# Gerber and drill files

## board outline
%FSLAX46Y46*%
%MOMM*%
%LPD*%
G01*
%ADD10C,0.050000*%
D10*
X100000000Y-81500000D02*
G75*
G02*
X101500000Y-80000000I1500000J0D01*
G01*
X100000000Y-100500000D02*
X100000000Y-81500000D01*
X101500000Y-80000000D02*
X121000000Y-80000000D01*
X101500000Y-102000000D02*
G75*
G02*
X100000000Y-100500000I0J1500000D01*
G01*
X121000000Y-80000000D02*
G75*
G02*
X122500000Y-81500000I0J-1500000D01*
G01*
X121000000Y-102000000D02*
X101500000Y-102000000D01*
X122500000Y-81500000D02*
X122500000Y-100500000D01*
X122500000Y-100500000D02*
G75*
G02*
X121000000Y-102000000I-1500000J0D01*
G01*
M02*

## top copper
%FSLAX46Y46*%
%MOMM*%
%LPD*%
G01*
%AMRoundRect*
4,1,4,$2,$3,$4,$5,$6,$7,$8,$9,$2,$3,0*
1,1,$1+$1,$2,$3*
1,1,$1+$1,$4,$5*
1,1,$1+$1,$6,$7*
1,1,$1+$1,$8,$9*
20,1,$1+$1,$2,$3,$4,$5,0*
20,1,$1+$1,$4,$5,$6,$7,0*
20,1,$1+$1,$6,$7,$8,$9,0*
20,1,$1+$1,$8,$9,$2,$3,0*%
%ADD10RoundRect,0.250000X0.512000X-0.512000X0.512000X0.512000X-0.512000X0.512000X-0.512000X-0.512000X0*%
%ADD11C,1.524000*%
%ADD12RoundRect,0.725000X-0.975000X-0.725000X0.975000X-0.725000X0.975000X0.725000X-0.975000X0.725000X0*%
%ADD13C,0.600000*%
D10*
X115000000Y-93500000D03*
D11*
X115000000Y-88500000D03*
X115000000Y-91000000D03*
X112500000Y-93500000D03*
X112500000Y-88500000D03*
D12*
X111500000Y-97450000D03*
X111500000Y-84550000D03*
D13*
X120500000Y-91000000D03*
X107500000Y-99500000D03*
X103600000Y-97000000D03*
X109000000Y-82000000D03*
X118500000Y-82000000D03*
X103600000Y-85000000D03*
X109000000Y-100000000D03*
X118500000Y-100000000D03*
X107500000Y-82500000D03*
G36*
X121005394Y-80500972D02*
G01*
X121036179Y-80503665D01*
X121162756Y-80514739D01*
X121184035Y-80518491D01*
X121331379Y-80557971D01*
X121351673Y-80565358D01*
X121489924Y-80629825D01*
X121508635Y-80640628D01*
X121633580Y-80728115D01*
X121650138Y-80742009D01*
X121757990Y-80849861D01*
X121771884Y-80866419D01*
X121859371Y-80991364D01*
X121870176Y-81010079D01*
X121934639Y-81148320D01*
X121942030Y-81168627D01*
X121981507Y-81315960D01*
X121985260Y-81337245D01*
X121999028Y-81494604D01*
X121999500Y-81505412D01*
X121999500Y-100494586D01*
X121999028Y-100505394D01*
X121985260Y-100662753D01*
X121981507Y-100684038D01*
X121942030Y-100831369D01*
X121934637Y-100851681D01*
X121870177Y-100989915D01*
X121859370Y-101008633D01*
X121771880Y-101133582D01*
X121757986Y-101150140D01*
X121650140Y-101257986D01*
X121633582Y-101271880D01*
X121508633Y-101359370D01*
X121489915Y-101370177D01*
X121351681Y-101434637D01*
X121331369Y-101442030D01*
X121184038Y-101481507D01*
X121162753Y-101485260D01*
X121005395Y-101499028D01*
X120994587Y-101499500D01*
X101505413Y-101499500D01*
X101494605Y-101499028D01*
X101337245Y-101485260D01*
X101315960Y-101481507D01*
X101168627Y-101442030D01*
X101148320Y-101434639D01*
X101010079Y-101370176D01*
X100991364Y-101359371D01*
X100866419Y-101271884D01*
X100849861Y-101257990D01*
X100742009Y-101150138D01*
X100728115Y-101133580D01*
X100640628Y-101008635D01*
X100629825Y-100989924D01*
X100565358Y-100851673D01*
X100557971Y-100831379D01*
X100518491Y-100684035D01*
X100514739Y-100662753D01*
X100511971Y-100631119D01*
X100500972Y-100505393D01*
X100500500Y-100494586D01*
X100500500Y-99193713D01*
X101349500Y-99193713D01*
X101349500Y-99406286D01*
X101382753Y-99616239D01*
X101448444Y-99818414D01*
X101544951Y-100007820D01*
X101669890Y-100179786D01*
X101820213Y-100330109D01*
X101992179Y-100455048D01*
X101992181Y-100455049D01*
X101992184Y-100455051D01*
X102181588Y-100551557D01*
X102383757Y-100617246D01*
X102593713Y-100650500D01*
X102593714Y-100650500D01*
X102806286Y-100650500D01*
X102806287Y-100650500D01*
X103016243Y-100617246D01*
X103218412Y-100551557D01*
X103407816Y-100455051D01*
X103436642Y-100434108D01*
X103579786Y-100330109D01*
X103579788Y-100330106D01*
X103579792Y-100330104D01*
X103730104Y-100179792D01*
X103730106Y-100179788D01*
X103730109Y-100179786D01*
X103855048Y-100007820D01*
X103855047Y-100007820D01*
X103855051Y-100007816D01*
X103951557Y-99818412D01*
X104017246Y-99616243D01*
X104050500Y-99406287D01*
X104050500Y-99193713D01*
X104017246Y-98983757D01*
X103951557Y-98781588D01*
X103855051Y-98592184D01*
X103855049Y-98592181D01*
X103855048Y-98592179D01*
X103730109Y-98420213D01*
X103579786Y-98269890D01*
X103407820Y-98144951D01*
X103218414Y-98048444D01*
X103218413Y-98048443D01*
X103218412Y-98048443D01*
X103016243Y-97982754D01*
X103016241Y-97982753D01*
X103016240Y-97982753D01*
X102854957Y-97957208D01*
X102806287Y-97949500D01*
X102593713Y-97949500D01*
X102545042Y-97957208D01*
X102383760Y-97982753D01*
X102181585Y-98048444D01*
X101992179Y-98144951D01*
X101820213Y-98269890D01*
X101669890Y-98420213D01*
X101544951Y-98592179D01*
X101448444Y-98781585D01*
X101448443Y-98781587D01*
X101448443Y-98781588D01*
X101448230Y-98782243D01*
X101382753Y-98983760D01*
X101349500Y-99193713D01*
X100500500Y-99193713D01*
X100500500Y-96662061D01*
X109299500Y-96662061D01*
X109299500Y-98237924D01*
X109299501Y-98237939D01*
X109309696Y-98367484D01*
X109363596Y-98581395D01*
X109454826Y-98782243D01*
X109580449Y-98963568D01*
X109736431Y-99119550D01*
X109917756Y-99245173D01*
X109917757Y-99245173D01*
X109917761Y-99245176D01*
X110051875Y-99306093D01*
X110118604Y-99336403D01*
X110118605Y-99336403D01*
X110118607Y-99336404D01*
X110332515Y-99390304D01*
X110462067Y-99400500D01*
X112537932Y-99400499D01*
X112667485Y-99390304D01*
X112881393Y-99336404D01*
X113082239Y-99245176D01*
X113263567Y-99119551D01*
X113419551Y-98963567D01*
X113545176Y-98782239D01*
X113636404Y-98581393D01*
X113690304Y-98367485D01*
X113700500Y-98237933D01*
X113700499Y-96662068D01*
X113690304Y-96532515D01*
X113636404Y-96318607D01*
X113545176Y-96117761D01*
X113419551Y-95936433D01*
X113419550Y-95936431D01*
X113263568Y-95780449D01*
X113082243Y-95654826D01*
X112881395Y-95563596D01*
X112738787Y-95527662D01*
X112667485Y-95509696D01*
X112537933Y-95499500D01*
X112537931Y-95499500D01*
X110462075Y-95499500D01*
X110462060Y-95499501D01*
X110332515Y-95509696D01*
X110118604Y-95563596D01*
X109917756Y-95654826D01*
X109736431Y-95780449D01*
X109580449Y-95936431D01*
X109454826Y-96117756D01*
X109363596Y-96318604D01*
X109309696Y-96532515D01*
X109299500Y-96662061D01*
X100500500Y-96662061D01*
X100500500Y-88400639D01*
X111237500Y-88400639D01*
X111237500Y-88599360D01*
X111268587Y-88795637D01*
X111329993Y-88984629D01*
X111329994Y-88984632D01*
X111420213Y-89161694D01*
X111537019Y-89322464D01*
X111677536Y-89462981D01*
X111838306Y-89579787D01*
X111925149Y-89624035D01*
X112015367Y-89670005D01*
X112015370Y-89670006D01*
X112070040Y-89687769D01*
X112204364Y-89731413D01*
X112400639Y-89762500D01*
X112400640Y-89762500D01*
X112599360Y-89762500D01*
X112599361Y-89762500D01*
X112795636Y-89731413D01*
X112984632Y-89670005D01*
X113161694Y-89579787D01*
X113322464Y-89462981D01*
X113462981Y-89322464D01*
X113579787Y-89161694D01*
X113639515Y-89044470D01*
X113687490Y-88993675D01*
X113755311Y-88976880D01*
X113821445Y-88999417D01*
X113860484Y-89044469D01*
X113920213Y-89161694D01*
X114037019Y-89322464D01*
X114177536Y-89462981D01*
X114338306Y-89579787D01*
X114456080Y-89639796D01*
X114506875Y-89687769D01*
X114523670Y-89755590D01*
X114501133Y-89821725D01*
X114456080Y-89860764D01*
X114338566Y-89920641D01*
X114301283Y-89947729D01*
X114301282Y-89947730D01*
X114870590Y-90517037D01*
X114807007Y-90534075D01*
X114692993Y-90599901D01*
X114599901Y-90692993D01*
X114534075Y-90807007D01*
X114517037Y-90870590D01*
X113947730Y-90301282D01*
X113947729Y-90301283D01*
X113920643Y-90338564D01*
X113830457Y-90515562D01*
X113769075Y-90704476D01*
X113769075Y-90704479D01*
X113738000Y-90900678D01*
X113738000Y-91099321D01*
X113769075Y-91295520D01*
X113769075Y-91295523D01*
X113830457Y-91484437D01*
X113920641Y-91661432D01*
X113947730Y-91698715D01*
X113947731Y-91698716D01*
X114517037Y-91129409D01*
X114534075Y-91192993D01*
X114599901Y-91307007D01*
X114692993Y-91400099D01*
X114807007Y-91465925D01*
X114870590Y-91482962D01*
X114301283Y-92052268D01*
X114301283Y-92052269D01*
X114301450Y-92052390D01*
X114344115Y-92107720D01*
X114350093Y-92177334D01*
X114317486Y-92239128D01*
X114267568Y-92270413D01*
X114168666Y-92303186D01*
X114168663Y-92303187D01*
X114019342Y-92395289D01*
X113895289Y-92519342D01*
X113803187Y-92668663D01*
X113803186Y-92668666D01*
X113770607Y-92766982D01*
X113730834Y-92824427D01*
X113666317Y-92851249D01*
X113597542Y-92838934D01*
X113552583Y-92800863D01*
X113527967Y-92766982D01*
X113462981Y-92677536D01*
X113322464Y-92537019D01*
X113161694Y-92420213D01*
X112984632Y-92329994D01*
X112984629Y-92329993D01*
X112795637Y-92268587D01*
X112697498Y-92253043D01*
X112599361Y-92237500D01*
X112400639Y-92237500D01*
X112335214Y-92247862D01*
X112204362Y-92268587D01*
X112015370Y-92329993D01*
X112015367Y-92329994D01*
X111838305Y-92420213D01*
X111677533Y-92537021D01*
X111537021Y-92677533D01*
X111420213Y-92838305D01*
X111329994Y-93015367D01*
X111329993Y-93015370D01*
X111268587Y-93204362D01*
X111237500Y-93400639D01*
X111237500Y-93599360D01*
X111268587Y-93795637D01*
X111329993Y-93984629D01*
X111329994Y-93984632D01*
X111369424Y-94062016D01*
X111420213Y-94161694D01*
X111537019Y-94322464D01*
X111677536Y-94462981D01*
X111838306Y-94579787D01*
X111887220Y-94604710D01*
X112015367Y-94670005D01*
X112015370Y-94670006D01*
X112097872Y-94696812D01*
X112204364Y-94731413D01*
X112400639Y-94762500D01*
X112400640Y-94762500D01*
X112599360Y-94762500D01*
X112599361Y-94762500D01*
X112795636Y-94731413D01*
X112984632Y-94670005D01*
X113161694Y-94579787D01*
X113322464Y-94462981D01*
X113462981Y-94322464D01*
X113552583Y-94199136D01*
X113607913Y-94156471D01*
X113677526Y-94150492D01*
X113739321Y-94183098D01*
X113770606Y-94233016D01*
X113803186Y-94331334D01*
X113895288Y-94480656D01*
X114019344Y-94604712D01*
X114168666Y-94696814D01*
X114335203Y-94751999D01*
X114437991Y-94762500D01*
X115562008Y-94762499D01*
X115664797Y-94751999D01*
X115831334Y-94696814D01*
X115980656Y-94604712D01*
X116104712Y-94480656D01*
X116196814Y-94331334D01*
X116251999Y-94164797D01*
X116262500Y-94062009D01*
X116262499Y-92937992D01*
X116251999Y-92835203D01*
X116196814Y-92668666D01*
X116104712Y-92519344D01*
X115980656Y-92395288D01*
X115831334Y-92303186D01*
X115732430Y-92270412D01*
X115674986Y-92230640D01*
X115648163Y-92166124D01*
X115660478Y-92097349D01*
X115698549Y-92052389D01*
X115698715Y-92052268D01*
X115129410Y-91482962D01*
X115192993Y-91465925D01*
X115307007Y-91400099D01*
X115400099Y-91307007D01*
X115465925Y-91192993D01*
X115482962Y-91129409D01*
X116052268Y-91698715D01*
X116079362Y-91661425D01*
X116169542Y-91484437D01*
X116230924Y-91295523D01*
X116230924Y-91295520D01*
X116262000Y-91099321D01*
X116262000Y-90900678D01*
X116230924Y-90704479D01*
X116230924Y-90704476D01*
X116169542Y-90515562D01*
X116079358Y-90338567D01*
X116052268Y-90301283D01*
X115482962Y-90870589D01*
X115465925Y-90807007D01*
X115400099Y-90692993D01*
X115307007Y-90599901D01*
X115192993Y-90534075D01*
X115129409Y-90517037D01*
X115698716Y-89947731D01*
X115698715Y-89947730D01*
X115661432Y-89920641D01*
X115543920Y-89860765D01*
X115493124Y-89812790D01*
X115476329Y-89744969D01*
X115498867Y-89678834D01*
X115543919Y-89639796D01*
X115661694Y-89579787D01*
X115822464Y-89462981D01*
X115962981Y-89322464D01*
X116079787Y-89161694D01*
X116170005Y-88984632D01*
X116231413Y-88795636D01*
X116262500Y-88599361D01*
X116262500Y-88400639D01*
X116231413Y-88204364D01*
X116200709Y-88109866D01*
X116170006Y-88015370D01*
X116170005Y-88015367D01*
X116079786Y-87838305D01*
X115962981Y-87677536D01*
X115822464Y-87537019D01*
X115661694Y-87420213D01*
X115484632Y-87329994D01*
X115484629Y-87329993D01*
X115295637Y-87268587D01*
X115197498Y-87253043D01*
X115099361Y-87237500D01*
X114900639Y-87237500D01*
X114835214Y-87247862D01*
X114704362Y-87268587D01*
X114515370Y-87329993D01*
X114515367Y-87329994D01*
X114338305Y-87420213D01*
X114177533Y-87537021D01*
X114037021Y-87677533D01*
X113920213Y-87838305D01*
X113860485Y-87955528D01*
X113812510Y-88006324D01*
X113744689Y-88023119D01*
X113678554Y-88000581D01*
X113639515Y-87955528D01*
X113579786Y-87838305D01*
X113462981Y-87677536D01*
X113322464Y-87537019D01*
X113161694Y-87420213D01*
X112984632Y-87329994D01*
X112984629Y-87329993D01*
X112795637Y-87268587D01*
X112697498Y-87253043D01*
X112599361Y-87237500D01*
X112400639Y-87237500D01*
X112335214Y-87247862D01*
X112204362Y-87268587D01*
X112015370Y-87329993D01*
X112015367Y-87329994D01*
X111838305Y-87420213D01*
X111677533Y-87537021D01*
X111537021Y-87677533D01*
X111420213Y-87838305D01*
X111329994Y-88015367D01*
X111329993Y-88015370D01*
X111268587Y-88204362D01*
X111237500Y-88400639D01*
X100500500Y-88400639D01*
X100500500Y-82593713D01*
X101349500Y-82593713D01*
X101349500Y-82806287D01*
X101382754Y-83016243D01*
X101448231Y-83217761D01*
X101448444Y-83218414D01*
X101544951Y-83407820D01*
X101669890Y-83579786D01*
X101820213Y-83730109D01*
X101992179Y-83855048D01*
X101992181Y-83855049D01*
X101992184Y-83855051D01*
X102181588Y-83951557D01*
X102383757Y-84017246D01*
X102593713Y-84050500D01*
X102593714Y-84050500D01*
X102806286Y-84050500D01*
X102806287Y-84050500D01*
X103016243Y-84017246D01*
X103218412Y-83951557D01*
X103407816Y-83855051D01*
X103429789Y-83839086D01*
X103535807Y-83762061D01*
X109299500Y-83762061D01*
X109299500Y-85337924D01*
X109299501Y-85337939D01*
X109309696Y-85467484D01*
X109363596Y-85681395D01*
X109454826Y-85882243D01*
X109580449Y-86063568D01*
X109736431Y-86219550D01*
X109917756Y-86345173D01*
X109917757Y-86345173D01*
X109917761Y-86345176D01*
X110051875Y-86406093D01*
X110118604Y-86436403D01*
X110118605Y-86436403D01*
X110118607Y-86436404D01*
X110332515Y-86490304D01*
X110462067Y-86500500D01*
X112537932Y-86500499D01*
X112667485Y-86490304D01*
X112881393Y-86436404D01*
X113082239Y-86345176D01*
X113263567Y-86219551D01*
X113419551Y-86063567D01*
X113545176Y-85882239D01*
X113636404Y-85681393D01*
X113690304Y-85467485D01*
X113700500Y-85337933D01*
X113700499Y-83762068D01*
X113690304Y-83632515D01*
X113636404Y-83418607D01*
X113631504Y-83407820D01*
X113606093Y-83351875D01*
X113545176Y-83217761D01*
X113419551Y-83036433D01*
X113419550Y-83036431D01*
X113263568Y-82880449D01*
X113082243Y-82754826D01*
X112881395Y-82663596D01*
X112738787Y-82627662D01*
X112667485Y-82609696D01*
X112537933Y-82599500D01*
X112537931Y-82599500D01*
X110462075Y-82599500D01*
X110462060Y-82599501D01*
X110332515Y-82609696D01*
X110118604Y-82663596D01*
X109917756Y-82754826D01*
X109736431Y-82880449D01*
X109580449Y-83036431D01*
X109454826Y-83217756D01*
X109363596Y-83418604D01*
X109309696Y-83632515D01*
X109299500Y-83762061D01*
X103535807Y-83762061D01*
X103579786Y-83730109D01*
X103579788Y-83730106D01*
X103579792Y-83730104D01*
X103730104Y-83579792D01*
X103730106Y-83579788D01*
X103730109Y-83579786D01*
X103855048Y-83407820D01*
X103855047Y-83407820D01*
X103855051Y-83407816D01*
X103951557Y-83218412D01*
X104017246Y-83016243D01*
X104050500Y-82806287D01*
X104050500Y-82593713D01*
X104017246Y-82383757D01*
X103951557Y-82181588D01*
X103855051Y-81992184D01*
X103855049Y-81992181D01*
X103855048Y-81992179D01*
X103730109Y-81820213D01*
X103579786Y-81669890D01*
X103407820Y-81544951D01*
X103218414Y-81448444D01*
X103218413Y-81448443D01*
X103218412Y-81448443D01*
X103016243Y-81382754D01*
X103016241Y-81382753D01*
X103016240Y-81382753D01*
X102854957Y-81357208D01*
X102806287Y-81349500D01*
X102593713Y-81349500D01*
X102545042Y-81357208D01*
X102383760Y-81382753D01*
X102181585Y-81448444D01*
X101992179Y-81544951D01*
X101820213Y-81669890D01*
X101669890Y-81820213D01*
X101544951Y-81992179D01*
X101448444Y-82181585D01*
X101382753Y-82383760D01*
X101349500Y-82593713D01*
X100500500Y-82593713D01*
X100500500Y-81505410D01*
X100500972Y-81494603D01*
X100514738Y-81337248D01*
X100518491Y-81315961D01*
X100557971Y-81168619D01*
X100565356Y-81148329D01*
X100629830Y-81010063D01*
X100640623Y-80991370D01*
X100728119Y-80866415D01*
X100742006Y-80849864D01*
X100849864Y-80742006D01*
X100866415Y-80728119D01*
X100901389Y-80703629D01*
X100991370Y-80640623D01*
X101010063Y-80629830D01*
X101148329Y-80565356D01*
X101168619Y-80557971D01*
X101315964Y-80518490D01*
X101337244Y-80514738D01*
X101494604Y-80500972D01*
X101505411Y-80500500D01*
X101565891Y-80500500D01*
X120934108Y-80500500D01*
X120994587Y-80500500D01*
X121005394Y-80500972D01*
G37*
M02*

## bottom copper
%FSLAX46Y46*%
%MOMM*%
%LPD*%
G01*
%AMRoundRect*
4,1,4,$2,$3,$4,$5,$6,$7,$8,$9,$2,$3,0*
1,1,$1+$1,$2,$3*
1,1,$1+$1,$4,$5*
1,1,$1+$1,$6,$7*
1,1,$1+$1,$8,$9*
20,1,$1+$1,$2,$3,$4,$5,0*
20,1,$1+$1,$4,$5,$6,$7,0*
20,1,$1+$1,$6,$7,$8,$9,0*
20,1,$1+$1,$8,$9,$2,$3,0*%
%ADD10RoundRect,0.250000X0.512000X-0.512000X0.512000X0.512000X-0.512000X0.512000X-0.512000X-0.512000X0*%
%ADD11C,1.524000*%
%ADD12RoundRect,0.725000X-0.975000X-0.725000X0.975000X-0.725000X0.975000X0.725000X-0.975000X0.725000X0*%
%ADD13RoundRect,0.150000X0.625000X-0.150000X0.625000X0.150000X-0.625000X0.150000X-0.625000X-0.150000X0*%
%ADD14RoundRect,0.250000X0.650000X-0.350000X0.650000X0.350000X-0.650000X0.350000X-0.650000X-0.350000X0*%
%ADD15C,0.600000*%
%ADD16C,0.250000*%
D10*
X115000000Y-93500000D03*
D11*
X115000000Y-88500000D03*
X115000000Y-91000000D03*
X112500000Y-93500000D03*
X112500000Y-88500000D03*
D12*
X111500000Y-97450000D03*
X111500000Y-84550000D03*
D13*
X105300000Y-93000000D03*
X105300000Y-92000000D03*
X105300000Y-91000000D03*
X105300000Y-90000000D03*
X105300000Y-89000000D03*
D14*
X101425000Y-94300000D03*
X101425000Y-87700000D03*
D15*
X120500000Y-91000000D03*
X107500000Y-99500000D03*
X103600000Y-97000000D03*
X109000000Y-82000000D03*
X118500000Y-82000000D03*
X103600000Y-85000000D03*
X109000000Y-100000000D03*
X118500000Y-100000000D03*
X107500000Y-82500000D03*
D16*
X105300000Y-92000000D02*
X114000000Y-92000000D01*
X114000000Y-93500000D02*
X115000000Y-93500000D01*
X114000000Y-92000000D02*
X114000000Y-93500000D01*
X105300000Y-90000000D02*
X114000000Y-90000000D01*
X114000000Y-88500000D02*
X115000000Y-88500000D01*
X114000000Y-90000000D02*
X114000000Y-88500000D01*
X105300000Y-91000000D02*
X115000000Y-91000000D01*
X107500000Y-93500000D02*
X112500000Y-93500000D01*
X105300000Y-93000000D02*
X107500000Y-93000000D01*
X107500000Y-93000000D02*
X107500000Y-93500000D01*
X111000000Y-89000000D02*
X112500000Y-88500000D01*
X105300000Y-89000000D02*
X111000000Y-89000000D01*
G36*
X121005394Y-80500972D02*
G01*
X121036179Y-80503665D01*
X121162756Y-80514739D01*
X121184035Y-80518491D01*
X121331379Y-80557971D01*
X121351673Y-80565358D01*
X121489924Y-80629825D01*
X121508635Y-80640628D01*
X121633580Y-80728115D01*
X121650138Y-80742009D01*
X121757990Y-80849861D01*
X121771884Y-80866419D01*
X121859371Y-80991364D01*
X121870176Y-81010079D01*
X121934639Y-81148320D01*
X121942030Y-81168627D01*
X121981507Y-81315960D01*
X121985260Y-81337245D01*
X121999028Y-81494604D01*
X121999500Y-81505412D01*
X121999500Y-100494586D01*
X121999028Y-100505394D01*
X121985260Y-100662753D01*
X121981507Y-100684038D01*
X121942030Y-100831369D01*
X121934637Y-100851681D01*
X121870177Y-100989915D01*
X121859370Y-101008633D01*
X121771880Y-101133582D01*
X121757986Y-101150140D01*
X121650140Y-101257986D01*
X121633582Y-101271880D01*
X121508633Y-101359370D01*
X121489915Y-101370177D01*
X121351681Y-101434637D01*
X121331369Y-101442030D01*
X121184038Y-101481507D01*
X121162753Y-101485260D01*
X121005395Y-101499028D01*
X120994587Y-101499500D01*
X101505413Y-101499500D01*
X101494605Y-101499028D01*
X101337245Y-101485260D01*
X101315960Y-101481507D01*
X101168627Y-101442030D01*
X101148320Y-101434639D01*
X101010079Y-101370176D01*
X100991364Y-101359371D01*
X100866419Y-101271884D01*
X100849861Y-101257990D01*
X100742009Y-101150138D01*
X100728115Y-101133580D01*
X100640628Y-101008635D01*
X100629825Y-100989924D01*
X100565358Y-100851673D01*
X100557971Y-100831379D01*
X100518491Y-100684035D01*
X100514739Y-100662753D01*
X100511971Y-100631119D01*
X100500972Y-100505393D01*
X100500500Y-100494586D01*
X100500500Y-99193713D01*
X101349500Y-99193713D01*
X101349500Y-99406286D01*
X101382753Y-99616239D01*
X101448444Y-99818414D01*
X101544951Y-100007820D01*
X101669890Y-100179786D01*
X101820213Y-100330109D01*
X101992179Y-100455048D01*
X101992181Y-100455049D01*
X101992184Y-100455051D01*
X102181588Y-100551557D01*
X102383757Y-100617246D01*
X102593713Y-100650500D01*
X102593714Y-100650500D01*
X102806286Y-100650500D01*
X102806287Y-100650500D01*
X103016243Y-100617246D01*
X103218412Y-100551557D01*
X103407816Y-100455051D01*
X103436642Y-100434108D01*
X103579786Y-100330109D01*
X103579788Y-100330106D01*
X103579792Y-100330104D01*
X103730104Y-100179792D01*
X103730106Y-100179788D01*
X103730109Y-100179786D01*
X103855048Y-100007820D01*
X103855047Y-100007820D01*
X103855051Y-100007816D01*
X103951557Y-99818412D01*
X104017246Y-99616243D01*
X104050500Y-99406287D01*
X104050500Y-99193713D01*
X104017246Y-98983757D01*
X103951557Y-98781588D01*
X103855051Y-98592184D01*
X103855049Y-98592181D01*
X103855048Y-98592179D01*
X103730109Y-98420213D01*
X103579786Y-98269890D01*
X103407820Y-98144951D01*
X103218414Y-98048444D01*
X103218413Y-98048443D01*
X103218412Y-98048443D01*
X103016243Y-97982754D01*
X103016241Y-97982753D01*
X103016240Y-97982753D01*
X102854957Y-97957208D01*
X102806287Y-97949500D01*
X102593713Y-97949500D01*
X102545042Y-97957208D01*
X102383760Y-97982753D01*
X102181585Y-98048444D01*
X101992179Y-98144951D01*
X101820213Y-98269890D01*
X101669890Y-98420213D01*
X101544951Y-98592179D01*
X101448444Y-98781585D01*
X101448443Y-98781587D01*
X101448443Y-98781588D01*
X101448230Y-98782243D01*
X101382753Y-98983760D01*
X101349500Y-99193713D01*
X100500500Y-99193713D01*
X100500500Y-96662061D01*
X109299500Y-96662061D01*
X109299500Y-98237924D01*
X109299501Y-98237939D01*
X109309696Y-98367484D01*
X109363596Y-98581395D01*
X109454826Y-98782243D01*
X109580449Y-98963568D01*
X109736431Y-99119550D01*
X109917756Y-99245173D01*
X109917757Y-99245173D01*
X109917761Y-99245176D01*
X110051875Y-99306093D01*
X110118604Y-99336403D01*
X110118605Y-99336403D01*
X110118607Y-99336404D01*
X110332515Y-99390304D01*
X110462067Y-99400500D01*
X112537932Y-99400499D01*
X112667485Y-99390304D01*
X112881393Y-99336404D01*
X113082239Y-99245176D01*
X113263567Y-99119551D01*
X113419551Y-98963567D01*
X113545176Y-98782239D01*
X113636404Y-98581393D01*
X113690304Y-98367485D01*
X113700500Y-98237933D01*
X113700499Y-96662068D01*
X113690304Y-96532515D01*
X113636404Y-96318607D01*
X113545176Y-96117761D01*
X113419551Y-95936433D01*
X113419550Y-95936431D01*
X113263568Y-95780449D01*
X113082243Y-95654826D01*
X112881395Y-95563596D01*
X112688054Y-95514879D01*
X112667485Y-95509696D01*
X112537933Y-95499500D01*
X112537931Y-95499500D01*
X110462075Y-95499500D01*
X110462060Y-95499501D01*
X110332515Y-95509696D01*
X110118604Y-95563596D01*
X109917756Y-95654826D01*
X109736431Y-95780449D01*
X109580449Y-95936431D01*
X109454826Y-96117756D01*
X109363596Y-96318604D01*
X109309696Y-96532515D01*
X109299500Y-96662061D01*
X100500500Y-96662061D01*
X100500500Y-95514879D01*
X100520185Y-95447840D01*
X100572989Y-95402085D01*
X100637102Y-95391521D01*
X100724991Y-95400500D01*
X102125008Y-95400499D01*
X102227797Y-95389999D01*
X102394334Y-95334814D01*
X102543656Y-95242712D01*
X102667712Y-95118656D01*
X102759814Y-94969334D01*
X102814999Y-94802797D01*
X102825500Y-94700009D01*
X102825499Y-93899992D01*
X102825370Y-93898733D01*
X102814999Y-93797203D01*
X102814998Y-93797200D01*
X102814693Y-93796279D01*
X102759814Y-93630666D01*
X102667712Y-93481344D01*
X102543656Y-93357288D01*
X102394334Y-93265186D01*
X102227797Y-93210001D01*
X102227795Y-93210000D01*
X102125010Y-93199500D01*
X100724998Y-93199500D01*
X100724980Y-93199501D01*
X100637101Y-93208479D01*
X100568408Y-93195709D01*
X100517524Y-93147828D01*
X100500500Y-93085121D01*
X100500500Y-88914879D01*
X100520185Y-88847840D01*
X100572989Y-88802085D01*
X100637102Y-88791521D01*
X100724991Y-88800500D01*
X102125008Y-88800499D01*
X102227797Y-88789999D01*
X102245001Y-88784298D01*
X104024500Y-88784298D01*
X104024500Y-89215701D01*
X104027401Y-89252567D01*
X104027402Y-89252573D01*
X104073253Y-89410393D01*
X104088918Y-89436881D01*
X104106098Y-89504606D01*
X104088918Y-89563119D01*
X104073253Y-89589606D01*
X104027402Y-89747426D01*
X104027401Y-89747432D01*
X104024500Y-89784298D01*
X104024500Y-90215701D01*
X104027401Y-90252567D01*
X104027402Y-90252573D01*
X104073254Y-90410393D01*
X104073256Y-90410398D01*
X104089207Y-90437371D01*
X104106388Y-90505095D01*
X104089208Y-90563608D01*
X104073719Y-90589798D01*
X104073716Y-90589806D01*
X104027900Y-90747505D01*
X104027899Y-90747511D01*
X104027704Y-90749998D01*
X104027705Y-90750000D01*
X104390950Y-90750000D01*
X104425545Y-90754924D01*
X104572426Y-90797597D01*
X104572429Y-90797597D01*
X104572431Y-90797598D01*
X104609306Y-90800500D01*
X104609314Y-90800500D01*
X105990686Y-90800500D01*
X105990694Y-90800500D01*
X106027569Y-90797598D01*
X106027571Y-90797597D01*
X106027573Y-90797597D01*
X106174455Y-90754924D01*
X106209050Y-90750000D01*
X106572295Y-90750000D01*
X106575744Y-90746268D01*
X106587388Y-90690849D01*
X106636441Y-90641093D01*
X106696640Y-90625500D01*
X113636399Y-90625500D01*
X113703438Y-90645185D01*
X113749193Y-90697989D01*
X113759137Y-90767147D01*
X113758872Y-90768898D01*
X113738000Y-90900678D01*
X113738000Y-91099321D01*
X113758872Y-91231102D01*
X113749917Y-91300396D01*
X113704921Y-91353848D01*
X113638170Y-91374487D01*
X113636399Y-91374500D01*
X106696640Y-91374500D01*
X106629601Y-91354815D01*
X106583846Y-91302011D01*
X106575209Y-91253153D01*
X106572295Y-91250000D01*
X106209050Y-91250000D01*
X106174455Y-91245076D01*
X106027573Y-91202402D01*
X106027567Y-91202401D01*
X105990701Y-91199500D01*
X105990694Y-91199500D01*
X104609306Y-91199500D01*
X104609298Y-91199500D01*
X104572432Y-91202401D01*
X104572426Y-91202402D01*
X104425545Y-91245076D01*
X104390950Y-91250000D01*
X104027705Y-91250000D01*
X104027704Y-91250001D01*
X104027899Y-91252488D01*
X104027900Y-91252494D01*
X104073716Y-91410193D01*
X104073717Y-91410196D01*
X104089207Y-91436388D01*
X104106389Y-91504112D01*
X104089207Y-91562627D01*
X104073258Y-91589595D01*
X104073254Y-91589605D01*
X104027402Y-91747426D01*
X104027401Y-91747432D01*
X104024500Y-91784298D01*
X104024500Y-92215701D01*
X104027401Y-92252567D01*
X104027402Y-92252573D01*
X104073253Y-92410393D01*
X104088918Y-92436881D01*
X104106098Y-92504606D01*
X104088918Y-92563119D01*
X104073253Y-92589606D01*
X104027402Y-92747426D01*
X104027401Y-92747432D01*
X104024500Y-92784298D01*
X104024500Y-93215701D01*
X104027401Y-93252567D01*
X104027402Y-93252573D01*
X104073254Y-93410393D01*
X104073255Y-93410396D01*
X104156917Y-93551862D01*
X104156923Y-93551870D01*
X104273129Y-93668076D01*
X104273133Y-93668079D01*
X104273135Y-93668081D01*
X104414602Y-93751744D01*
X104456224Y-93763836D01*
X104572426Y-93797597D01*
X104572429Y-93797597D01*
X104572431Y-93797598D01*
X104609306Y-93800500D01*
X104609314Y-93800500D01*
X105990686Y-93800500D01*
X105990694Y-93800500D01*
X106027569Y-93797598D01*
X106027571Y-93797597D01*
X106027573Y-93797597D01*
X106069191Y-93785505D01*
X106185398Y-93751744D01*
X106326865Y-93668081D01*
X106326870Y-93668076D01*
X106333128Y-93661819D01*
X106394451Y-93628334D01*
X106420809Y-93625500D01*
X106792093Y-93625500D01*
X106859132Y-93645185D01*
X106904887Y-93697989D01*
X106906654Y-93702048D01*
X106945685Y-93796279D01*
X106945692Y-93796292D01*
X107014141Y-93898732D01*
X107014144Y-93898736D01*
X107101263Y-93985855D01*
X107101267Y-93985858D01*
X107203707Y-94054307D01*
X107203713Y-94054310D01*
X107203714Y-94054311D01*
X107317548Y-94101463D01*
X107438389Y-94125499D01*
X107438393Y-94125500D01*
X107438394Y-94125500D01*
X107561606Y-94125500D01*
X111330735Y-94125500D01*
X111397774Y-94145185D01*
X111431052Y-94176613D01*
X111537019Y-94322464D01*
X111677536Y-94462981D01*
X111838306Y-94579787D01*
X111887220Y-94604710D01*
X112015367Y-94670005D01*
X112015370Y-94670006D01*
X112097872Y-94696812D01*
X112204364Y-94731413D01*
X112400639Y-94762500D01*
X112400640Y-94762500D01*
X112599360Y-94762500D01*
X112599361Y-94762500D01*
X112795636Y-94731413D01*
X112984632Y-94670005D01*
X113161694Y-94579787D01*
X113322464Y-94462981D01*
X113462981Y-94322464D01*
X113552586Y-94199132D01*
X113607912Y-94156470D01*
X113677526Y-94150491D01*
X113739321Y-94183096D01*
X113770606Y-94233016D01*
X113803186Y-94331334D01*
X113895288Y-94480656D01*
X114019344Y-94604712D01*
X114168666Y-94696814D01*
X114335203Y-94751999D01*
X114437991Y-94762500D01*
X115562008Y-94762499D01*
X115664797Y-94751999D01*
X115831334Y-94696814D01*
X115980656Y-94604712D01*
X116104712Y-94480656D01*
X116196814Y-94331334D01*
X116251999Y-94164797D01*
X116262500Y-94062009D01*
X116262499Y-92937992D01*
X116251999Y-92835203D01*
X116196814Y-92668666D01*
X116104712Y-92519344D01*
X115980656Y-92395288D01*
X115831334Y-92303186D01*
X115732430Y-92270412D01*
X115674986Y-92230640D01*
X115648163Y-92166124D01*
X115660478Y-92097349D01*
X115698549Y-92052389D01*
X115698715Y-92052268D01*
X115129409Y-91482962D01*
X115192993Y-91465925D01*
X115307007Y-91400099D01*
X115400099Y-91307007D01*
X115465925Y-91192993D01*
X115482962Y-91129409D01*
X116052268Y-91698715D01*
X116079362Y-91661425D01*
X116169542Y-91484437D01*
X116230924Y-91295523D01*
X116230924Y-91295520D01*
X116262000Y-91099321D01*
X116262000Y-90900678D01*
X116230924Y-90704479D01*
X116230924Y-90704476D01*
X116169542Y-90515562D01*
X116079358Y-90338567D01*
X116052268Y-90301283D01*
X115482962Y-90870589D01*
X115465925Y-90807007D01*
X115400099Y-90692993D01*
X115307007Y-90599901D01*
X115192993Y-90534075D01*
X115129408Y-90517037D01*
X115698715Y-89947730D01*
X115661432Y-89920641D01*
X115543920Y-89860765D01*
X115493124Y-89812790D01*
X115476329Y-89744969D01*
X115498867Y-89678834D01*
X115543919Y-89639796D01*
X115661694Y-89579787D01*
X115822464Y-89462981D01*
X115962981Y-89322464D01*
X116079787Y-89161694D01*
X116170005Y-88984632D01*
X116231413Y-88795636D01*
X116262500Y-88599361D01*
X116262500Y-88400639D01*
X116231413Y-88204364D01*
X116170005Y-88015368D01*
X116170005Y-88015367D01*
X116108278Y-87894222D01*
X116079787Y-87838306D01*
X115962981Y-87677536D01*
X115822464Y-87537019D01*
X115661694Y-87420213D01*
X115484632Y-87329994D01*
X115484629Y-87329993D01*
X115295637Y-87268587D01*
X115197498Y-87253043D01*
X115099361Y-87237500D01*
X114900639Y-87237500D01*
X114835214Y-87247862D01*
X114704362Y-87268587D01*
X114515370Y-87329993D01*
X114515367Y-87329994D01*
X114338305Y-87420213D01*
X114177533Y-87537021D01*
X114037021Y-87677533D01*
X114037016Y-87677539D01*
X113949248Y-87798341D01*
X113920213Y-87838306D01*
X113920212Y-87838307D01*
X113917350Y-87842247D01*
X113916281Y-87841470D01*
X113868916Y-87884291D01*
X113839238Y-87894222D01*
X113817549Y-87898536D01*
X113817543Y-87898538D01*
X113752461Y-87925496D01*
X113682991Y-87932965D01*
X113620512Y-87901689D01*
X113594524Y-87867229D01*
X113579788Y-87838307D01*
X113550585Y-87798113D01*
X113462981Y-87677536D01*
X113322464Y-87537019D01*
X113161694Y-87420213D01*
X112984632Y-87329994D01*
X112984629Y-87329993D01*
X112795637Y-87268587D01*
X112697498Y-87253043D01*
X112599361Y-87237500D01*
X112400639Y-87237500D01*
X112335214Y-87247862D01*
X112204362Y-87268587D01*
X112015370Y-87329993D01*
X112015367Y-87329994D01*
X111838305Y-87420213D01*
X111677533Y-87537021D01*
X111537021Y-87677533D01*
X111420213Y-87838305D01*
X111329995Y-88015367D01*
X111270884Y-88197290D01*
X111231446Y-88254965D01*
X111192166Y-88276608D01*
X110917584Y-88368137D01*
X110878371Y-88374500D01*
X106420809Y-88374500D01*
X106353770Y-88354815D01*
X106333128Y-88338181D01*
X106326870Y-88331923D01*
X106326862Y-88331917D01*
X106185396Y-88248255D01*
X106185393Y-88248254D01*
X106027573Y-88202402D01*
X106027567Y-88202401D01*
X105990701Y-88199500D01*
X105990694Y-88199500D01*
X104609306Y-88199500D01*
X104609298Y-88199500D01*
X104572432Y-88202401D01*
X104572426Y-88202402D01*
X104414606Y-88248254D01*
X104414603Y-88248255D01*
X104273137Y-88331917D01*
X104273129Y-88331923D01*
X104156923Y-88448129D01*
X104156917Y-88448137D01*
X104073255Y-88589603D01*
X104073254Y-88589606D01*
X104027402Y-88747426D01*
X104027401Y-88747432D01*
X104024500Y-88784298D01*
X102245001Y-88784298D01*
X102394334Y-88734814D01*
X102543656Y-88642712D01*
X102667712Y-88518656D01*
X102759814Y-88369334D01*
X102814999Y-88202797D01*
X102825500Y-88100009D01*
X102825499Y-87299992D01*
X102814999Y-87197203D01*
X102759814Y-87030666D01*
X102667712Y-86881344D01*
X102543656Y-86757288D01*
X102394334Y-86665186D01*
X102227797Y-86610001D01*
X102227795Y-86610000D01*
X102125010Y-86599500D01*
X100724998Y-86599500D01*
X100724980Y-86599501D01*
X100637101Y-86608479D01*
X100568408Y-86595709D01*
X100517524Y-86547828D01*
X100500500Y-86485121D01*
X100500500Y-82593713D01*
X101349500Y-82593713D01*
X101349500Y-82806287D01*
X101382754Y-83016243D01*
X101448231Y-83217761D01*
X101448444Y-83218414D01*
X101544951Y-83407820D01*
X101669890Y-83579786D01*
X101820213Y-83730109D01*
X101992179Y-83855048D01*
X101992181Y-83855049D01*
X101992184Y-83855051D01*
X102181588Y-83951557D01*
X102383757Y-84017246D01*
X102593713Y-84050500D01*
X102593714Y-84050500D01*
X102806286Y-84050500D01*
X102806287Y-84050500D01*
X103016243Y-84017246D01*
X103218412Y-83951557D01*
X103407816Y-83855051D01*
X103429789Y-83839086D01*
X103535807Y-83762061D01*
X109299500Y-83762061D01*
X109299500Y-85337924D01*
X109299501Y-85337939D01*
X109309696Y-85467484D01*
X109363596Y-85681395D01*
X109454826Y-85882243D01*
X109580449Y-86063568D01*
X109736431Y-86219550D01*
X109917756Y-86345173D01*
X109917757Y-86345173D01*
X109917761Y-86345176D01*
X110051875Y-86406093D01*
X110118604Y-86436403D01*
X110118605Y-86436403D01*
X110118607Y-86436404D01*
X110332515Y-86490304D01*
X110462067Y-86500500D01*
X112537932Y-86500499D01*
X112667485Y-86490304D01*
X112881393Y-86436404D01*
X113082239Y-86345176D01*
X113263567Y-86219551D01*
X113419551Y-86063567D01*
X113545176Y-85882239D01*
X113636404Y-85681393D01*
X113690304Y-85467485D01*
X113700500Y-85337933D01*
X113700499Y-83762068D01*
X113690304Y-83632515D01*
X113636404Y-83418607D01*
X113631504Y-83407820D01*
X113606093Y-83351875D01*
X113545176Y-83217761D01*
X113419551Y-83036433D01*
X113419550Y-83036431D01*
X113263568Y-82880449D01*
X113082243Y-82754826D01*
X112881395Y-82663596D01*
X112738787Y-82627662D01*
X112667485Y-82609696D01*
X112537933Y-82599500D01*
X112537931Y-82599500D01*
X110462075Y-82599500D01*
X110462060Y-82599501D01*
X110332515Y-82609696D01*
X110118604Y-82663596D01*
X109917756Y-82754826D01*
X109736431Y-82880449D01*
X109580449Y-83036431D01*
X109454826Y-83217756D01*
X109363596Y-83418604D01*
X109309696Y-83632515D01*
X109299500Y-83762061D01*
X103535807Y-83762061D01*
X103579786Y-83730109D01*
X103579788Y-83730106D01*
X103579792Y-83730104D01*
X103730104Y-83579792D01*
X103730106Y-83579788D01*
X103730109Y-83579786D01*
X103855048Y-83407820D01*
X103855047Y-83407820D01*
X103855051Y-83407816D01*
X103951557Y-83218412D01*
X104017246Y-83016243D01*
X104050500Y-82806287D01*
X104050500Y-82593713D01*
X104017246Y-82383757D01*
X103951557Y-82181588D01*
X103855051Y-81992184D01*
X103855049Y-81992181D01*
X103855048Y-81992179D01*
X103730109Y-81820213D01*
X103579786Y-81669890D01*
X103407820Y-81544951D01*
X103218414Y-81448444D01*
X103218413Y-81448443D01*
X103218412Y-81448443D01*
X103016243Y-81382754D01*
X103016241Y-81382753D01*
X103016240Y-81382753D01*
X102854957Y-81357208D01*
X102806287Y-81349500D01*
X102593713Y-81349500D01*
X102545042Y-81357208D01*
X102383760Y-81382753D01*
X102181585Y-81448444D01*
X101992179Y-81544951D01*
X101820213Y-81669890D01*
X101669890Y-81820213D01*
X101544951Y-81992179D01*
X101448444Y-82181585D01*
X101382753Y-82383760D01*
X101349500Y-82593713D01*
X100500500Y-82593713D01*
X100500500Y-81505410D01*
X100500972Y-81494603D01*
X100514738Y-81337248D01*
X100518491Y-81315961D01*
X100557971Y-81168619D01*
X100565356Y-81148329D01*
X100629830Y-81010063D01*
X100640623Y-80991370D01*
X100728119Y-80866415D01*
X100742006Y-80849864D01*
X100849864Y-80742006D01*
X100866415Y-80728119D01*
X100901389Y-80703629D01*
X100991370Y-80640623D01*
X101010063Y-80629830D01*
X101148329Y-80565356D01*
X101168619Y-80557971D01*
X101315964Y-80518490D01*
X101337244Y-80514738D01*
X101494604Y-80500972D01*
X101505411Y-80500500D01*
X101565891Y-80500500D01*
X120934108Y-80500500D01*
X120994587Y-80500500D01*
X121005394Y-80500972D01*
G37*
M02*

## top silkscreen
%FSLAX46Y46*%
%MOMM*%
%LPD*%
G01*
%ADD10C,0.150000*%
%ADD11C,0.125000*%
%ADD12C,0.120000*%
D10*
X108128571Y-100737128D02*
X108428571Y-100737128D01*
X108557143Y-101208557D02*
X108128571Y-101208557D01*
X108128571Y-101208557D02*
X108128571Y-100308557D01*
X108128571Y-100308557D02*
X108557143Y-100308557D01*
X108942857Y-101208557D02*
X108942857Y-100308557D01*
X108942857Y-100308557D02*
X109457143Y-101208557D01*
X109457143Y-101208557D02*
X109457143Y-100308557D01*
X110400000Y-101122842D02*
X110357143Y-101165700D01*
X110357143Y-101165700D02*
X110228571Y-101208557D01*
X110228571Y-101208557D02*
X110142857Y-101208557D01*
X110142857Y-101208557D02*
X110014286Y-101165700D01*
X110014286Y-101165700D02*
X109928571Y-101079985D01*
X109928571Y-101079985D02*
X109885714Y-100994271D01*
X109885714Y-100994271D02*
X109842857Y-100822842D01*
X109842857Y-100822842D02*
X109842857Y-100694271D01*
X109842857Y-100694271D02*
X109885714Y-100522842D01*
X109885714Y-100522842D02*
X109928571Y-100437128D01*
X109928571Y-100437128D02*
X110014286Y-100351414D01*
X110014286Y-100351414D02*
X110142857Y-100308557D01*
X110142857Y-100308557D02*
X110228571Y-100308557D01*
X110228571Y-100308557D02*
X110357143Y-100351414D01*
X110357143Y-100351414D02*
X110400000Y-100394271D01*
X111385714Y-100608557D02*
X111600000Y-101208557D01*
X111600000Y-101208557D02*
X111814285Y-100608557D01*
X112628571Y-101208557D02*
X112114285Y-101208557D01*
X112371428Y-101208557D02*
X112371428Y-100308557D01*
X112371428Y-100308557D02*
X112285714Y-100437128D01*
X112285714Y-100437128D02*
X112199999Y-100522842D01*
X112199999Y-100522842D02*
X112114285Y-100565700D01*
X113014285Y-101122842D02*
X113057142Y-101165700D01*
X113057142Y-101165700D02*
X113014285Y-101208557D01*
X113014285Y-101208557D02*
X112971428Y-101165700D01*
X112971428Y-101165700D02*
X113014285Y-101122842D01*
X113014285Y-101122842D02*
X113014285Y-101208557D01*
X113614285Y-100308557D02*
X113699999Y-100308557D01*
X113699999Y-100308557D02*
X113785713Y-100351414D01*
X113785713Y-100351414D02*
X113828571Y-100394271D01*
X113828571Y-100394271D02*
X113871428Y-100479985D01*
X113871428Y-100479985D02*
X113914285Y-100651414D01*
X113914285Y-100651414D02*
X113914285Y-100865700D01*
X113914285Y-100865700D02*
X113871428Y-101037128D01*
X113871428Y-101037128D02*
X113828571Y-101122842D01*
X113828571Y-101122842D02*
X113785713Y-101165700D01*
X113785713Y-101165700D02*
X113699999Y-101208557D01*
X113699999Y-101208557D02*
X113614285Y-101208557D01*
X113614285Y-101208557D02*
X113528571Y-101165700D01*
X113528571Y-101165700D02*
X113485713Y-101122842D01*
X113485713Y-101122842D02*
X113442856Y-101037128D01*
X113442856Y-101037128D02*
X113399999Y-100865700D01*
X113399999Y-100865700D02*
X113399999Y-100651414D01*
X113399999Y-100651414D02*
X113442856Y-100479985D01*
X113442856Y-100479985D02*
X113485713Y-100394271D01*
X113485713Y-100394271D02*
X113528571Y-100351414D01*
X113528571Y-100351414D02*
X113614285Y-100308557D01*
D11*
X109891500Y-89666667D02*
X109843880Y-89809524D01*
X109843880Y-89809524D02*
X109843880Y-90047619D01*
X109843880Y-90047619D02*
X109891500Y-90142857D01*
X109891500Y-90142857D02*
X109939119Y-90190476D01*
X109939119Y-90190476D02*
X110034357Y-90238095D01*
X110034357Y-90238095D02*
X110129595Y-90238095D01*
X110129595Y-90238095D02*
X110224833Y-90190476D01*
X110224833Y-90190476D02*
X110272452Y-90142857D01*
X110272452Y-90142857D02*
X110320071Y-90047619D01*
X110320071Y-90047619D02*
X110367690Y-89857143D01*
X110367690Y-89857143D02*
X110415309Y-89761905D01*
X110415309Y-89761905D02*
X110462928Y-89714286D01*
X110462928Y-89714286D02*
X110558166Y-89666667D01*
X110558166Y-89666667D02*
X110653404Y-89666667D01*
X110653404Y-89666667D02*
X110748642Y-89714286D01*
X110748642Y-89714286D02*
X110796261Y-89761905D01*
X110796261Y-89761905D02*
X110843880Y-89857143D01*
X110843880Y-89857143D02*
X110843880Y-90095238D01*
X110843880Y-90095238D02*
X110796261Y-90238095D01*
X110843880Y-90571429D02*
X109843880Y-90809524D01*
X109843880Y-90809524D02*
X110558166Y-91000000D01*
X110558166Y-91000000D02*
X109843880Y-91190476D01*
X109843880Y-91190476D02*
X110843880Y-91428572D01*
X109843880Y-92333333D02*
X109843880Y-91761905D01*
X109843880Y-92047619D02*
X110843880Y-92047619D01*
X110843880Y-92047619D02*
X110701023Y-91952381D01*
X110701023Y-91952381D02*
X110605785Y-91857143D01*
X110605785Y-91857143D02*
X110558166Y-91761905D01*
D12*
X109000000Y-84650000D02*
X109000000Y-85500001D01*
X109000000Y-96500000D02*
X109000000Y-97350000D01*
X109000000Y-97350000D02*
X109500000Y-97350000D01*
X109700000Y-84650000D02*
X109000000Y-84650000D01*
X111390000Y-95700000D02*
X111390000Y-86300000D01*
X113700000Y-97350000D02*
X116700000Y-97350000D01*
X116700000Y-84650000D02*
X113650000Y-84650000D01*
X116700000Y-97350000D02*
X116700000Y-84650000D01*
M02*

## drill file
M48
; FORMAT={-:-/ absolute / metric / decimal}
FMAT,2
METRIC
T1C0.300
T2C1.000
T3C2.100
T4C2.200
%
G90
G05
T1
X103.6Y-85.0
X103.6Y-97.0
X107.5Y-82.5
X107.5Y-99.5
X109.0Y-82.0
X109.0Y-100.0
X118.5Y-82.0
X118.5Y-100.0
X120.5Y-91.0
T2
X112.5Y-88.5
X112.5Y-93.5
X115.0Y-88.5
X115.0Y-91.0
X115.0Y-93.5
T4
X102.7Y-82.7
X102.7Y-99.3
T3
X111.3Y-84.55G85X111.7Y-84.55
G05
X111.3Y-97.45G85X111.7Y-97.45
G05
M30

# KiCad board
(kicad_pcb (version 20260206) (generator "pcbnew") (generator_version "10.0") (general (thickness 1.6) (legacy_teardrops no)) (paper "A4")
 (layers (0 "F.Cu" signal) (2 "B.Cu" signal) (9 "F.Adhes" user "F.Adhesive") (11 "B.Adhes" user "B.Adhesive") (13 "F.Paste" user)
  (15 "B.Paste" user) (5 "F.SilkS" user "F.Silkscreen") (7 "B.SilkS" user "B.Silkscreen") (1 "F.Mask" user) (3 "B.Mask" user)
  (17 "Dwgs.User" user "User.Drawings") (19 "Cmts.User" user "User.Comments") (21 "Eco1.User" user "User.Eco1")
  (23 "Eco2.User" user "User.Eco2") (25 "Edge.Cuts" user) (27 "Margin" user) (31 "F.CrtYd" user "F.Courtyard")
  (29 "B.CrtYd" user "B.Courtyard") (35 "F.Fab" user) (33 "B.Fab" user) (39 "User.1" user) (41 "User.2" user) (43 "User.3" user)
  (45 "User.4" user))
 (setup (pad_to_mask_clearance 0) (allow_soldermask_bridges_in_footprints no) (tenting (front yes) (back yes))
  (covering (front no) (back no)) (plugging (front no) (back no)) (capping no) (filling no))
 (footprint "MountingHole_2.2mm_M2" (layer "F.Cu") (at 102.7 99.3)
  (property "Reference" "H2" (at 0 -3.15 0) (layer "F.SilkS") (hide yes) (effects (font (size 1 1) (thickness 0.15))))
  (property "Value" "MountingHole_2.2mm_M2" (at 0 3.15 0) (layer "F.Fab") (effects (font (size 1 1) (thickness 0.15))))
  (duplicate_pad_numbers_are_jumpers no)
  (pad "" np_thru_hole circle (at 0 0) (size 2.2 2.2) (drill 2.2) (layers "*.Cu" "*.Mask")))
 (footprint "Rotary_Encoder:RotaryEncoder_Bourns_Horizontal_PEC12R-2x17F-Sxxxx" (layer "F.Cu") (at 115 93.5 180)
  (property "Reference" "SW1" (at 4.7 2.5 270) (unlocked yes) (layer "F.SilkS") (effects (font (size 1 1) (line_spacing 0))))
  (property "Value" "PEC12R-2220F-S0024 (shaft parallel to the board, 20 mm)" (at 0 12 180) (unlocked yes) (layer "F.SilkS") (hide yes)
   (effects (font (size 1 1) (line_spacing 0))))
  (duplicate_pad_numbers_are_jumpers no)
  (fp_line (start 6 8.85) (end 6 7.999999) (stroke (width 0.12) (type solid)) (layer "F.SilkS"))
  (fp_line (start 6 -3) (end 6 -3.85) (stroke (width 0.12) (type solid)) (layer "F.SilkS"))
  (fp_line (start 6 -3.85) (end 5.5 -3.85) (stroke (width 0.12) (type solid)) (layer "F.SilkS"))
  (fp_line (start 5.3 8.85) (end 6 8.85) (stroke (width 0.12) (type solid)) (layer "F.SilkS"))
  (fp_line (start 3.61 -2.2) (end 3.61 7.2) (stroke (width 0.12) (type solid)) (layer "F.SilkS"))
  (fp_line (start 1.3 -3.85) (end -1.7 -3.85) (stroke (width 0.12) (type solid)) (layer "F.SilkS"))
  (fp_line (start -1.7 8.85) (end 1.35 8.85) (stroke (width 0.12) (type solid)) (layer "F.SilkS"))
  (fp_line (start -1.7 -3.85) (end -1.7 8.85) (stroke (width 0.12) (type solid)) (layer "F.SilkS"))
  (pad "A" thru_hole roundrect (at 0 0 90) (size 1.524 1.524) (drill 1) (layers "*.Cu" "*.Mask") (remove_unused_layers no)
   (roundrect_rratio 0.1640419948) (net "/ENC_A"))
  (pad "B" thru_hole circle (at 0 5 90) (size 1.524 1.524) (drill 1) (layers "*.Cu" "*.Mask") (remove_unused_layers no) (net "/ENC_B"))
  (pad "C" thru_hole circle (at 0 2.5 90) (size 1.524 1.524) (drill 1) (layers "*.Cu" "*.Mask") (remove_unused_layers no) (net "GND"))
  (pad "S1" thru_hole circle (at 2.5 0 90) (size 1.524 1.524) (drill 1) (layers "*.Cu" "*.Mask") (remove_unused_layers no) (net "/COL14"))
  (pad "S2" thru_hole circle (at 2.5 5 90) (size 1.524 1.524) (drill 1) (layers "*.Cu" "*.Mask") (remove_unused_layers no) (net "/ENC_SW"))
  (pad "SH" thru_hole roundrect (at 3.5 -3.95) (size 3.4 2.9) (drill oval 2.5 2.1) (layers "*.Cu" "*.Mask") (remove_unused_layers no)
   (roundrect_rratio 0.25))
  (pad "SH" thru_hole roundrect (at 3.5 8.95) (size 3.4 2.9) (drill oval 2.5 2.1) (layers "*.Cu" "*.Mask") (remove_unused_layers no)
   (roundrect_rratio 0.25)))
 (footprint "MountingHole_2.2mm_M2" (layer "F.Cu") (at 102.7 82.7)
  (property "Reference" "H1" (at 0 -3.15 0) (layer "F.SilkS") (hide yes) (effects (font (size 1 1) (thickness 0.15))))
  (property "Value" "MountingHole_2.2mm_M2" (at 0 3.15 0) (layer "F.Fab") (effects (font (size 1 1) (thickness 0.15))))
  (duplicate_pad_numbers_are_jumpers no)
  (pad "" np_thru_hole circle (at 0 0) (size 2.2 2.2) (drill 2.2) (layers "*.Cu" "*.Mask")))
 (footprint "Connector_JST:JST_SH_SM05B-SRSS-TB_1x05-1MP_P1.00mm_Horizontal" (layer "B.Cu") (at 103.3 91 90)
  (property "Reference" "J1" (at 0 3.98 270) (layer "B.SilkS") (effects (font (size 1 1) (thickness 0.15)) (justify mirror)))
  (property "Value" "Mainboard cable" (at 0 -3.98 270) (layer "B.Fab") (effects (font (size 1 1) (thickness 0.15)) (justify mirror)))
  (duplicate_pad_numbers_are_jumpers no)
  (pad "1" smd roundrect (at -2 2 90) (size 0.6 1.55) (layers "B.Cu" "B.Mask" "B.Paste") (roundrect_rratio 0.25) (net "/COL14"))
  (pad "2" smd roundrect (at -1 2 90) (size 0.6 1.55) (layers "B.Cu" "B.Mask" "B.Paste") (roundrect_rratio 0.25) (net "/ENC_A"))
  (pad "3" smd roundrect (at 0 2 90) (size 0.6 1.55) (layers "B.Cu" "B.Mask" "B.Paste") (roundrect_rratio 0.25) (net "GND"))
  (pad "4" smd roundrect (at 1 2 90) (size 0.6 1.55) (layers "B.Cu" "B.Mask" "B.Paste") (roundrect_rratio 0.25) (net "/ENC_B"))
  (pad "5" smd roundrect (at 2 2 90) (size 0.6 1.55) (layers "B.Cu" "B.Mask" "B.Paste") (roundrect_rratio 0.25) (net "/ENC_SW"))
  (pad "MP" smd roundrect (at -3.3 -1.875 90) (size 1.2 1.8) (layers "B.Cu" "B.Mask" "B.Paste") (roundrect_rratio 0.208333))
  (pad "MP" smd roundrect (at 3.3 -1.875 90) (size 1.2 1.8) (layers "B.Cu" "B.Mask" "B.Paste") (roundrect_rratio 0.208333)))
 (gr_arc (start 100 81.5) (mid 100.439339 80.439339) (end 101.5 80) (stroke (width 0.05) (type default)) (layer "Edge.Cuts"))
 (gr_line (start 100 100.5) (end 100 81.5) (stroke (width 0.05) (type default)) (layer "Edge.Cuts"))
 (gr_line (start 101.5 80) (end 121 80) (stroke (width 0.05) (type default)) (layer "Edge.Cuts"))
 (gr_arc (start 101.5 102) (mid 100.439339 101.56066) (end 100 100.5) (stroke (width 0.05) (type default)) (layer "Edge.Cuts"))
 (gr_arc (start 121 80) (mid 122.06066 80.439339) (end 122.5 81.5) (stroke (width 0.05) (type default)) (layer "Edge.Cuts"))
 (gr_line (start 121 102) (end 101.5 102) (stroke (width 0.05) (type default)) (layer "Edge.Cuts"))
 (gr_line (start 122.5 81.5) (end 122.5 100.5) (stroke (width 0.05) (type default)) (layer "Edge.Cuts"))
 (gr_arc (start 122.5 100.5) (mid 122.06066 101.56066) (end 121 102) (stroke (width 0.05) (type default)) (layer "Edge.Cuts"))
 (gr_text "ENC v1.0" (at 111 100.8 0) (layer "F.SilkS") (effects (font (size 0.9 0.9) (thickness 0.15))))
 (segment (start 105.3 92) (end 114 92) (width 0.25) (layer "B.Cu") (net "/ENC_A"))
 (segment (start 114 93.5) (end 115 93.5) (width 0.25) (layer "B.Cu") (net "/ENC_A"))
 (segment (start 114 92) (end 114 93.5) (width 0.25) (layer "B.Cu") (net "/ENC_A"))
 (segment (start 105.3 90) (end 114 90) (width 0.25) (layer "B.Cu") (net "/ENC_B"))
 (segment (start 114 88.5) (end 115 88.5) (width 0.25) (layer "B.Cu") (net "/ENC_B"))
 (segment (start 114 90) (end 114 88.5) (width 0.25) (layer "B.Cu") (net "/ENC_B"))
 (via (at 120.5 91) (size 0.6) (drill 0.3) (layers "F.Cu" "B.Cu") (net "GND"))
 (via (at 107.5 99.5) (size 0.6) (drill 0.3) (layers "F.Cu" "B.Cu") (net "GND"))
 (via (at 103.6 97) (size 0.6) (drill 0.3) (layers "F.Cu" "B.Cu") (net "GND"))
 (via (at 109 82) (size 0.6) (drill 0.3) (layers "F.Cu" "B.Cu") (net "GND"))
 (via (at 118.5 82) (size 0.6) (drill 0.3) (layers "F.Cu" "B.Cu") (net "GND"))
 (via (at 103.6 85) (size 0.6) (drill 0.3) (layers "F.Cu" "B.Cu") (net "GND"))
 (via (at 109 100) (size 0.6) (drill 0.3) (layers "F.Cu" "B.Cu") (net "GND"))
 (via (at 118.5 100) (size 0.6) (drill 0.3) (layers "F.Cu" "B.Cu") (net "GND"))
 (via (at 107.5 82.5) (size 0.6) (drill 0.3) (layers "F.Cu" "B.Cu") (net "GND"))
 (segment (start 105.3 91) (end 115 91) (width 0.25) (layer "B.Cu") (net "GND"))
 (segment (start 107.5 93.5) (end 112.5 93.5) (width 0.25) (layer "B.Cu") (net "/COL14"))
 (segment (start 105.3 93) (end 107.5 93) (width 0.25) (layer "B.Cu") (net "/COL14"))
 (segment (start 107.5 93) (end 107.5 93.5) (width 0.25) (layer "B.Cu") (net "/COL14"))
 (segment (start 111 89) (end 112.5 88.5) (width 0.25) (layer "B.Cu") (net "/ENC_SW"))
 (segment (start 105.3 89) (end 111 89) (width 0.25) (layer "B.Cu") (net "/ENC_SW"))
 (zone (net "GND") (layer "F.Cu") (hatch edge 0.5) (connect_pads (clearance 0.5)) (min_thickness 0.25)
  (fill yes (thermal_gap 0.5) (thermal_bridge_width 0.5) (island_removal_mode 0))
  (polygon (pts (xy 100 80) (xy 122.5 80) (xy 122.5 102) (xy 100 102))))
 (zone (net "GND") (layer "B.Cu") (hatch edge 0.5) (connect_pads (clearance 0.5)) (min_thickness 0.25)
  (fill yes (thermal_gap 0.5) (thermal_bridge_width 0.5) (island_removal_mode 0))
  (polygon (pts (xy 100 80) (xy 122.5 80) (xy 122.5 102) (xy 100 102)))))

